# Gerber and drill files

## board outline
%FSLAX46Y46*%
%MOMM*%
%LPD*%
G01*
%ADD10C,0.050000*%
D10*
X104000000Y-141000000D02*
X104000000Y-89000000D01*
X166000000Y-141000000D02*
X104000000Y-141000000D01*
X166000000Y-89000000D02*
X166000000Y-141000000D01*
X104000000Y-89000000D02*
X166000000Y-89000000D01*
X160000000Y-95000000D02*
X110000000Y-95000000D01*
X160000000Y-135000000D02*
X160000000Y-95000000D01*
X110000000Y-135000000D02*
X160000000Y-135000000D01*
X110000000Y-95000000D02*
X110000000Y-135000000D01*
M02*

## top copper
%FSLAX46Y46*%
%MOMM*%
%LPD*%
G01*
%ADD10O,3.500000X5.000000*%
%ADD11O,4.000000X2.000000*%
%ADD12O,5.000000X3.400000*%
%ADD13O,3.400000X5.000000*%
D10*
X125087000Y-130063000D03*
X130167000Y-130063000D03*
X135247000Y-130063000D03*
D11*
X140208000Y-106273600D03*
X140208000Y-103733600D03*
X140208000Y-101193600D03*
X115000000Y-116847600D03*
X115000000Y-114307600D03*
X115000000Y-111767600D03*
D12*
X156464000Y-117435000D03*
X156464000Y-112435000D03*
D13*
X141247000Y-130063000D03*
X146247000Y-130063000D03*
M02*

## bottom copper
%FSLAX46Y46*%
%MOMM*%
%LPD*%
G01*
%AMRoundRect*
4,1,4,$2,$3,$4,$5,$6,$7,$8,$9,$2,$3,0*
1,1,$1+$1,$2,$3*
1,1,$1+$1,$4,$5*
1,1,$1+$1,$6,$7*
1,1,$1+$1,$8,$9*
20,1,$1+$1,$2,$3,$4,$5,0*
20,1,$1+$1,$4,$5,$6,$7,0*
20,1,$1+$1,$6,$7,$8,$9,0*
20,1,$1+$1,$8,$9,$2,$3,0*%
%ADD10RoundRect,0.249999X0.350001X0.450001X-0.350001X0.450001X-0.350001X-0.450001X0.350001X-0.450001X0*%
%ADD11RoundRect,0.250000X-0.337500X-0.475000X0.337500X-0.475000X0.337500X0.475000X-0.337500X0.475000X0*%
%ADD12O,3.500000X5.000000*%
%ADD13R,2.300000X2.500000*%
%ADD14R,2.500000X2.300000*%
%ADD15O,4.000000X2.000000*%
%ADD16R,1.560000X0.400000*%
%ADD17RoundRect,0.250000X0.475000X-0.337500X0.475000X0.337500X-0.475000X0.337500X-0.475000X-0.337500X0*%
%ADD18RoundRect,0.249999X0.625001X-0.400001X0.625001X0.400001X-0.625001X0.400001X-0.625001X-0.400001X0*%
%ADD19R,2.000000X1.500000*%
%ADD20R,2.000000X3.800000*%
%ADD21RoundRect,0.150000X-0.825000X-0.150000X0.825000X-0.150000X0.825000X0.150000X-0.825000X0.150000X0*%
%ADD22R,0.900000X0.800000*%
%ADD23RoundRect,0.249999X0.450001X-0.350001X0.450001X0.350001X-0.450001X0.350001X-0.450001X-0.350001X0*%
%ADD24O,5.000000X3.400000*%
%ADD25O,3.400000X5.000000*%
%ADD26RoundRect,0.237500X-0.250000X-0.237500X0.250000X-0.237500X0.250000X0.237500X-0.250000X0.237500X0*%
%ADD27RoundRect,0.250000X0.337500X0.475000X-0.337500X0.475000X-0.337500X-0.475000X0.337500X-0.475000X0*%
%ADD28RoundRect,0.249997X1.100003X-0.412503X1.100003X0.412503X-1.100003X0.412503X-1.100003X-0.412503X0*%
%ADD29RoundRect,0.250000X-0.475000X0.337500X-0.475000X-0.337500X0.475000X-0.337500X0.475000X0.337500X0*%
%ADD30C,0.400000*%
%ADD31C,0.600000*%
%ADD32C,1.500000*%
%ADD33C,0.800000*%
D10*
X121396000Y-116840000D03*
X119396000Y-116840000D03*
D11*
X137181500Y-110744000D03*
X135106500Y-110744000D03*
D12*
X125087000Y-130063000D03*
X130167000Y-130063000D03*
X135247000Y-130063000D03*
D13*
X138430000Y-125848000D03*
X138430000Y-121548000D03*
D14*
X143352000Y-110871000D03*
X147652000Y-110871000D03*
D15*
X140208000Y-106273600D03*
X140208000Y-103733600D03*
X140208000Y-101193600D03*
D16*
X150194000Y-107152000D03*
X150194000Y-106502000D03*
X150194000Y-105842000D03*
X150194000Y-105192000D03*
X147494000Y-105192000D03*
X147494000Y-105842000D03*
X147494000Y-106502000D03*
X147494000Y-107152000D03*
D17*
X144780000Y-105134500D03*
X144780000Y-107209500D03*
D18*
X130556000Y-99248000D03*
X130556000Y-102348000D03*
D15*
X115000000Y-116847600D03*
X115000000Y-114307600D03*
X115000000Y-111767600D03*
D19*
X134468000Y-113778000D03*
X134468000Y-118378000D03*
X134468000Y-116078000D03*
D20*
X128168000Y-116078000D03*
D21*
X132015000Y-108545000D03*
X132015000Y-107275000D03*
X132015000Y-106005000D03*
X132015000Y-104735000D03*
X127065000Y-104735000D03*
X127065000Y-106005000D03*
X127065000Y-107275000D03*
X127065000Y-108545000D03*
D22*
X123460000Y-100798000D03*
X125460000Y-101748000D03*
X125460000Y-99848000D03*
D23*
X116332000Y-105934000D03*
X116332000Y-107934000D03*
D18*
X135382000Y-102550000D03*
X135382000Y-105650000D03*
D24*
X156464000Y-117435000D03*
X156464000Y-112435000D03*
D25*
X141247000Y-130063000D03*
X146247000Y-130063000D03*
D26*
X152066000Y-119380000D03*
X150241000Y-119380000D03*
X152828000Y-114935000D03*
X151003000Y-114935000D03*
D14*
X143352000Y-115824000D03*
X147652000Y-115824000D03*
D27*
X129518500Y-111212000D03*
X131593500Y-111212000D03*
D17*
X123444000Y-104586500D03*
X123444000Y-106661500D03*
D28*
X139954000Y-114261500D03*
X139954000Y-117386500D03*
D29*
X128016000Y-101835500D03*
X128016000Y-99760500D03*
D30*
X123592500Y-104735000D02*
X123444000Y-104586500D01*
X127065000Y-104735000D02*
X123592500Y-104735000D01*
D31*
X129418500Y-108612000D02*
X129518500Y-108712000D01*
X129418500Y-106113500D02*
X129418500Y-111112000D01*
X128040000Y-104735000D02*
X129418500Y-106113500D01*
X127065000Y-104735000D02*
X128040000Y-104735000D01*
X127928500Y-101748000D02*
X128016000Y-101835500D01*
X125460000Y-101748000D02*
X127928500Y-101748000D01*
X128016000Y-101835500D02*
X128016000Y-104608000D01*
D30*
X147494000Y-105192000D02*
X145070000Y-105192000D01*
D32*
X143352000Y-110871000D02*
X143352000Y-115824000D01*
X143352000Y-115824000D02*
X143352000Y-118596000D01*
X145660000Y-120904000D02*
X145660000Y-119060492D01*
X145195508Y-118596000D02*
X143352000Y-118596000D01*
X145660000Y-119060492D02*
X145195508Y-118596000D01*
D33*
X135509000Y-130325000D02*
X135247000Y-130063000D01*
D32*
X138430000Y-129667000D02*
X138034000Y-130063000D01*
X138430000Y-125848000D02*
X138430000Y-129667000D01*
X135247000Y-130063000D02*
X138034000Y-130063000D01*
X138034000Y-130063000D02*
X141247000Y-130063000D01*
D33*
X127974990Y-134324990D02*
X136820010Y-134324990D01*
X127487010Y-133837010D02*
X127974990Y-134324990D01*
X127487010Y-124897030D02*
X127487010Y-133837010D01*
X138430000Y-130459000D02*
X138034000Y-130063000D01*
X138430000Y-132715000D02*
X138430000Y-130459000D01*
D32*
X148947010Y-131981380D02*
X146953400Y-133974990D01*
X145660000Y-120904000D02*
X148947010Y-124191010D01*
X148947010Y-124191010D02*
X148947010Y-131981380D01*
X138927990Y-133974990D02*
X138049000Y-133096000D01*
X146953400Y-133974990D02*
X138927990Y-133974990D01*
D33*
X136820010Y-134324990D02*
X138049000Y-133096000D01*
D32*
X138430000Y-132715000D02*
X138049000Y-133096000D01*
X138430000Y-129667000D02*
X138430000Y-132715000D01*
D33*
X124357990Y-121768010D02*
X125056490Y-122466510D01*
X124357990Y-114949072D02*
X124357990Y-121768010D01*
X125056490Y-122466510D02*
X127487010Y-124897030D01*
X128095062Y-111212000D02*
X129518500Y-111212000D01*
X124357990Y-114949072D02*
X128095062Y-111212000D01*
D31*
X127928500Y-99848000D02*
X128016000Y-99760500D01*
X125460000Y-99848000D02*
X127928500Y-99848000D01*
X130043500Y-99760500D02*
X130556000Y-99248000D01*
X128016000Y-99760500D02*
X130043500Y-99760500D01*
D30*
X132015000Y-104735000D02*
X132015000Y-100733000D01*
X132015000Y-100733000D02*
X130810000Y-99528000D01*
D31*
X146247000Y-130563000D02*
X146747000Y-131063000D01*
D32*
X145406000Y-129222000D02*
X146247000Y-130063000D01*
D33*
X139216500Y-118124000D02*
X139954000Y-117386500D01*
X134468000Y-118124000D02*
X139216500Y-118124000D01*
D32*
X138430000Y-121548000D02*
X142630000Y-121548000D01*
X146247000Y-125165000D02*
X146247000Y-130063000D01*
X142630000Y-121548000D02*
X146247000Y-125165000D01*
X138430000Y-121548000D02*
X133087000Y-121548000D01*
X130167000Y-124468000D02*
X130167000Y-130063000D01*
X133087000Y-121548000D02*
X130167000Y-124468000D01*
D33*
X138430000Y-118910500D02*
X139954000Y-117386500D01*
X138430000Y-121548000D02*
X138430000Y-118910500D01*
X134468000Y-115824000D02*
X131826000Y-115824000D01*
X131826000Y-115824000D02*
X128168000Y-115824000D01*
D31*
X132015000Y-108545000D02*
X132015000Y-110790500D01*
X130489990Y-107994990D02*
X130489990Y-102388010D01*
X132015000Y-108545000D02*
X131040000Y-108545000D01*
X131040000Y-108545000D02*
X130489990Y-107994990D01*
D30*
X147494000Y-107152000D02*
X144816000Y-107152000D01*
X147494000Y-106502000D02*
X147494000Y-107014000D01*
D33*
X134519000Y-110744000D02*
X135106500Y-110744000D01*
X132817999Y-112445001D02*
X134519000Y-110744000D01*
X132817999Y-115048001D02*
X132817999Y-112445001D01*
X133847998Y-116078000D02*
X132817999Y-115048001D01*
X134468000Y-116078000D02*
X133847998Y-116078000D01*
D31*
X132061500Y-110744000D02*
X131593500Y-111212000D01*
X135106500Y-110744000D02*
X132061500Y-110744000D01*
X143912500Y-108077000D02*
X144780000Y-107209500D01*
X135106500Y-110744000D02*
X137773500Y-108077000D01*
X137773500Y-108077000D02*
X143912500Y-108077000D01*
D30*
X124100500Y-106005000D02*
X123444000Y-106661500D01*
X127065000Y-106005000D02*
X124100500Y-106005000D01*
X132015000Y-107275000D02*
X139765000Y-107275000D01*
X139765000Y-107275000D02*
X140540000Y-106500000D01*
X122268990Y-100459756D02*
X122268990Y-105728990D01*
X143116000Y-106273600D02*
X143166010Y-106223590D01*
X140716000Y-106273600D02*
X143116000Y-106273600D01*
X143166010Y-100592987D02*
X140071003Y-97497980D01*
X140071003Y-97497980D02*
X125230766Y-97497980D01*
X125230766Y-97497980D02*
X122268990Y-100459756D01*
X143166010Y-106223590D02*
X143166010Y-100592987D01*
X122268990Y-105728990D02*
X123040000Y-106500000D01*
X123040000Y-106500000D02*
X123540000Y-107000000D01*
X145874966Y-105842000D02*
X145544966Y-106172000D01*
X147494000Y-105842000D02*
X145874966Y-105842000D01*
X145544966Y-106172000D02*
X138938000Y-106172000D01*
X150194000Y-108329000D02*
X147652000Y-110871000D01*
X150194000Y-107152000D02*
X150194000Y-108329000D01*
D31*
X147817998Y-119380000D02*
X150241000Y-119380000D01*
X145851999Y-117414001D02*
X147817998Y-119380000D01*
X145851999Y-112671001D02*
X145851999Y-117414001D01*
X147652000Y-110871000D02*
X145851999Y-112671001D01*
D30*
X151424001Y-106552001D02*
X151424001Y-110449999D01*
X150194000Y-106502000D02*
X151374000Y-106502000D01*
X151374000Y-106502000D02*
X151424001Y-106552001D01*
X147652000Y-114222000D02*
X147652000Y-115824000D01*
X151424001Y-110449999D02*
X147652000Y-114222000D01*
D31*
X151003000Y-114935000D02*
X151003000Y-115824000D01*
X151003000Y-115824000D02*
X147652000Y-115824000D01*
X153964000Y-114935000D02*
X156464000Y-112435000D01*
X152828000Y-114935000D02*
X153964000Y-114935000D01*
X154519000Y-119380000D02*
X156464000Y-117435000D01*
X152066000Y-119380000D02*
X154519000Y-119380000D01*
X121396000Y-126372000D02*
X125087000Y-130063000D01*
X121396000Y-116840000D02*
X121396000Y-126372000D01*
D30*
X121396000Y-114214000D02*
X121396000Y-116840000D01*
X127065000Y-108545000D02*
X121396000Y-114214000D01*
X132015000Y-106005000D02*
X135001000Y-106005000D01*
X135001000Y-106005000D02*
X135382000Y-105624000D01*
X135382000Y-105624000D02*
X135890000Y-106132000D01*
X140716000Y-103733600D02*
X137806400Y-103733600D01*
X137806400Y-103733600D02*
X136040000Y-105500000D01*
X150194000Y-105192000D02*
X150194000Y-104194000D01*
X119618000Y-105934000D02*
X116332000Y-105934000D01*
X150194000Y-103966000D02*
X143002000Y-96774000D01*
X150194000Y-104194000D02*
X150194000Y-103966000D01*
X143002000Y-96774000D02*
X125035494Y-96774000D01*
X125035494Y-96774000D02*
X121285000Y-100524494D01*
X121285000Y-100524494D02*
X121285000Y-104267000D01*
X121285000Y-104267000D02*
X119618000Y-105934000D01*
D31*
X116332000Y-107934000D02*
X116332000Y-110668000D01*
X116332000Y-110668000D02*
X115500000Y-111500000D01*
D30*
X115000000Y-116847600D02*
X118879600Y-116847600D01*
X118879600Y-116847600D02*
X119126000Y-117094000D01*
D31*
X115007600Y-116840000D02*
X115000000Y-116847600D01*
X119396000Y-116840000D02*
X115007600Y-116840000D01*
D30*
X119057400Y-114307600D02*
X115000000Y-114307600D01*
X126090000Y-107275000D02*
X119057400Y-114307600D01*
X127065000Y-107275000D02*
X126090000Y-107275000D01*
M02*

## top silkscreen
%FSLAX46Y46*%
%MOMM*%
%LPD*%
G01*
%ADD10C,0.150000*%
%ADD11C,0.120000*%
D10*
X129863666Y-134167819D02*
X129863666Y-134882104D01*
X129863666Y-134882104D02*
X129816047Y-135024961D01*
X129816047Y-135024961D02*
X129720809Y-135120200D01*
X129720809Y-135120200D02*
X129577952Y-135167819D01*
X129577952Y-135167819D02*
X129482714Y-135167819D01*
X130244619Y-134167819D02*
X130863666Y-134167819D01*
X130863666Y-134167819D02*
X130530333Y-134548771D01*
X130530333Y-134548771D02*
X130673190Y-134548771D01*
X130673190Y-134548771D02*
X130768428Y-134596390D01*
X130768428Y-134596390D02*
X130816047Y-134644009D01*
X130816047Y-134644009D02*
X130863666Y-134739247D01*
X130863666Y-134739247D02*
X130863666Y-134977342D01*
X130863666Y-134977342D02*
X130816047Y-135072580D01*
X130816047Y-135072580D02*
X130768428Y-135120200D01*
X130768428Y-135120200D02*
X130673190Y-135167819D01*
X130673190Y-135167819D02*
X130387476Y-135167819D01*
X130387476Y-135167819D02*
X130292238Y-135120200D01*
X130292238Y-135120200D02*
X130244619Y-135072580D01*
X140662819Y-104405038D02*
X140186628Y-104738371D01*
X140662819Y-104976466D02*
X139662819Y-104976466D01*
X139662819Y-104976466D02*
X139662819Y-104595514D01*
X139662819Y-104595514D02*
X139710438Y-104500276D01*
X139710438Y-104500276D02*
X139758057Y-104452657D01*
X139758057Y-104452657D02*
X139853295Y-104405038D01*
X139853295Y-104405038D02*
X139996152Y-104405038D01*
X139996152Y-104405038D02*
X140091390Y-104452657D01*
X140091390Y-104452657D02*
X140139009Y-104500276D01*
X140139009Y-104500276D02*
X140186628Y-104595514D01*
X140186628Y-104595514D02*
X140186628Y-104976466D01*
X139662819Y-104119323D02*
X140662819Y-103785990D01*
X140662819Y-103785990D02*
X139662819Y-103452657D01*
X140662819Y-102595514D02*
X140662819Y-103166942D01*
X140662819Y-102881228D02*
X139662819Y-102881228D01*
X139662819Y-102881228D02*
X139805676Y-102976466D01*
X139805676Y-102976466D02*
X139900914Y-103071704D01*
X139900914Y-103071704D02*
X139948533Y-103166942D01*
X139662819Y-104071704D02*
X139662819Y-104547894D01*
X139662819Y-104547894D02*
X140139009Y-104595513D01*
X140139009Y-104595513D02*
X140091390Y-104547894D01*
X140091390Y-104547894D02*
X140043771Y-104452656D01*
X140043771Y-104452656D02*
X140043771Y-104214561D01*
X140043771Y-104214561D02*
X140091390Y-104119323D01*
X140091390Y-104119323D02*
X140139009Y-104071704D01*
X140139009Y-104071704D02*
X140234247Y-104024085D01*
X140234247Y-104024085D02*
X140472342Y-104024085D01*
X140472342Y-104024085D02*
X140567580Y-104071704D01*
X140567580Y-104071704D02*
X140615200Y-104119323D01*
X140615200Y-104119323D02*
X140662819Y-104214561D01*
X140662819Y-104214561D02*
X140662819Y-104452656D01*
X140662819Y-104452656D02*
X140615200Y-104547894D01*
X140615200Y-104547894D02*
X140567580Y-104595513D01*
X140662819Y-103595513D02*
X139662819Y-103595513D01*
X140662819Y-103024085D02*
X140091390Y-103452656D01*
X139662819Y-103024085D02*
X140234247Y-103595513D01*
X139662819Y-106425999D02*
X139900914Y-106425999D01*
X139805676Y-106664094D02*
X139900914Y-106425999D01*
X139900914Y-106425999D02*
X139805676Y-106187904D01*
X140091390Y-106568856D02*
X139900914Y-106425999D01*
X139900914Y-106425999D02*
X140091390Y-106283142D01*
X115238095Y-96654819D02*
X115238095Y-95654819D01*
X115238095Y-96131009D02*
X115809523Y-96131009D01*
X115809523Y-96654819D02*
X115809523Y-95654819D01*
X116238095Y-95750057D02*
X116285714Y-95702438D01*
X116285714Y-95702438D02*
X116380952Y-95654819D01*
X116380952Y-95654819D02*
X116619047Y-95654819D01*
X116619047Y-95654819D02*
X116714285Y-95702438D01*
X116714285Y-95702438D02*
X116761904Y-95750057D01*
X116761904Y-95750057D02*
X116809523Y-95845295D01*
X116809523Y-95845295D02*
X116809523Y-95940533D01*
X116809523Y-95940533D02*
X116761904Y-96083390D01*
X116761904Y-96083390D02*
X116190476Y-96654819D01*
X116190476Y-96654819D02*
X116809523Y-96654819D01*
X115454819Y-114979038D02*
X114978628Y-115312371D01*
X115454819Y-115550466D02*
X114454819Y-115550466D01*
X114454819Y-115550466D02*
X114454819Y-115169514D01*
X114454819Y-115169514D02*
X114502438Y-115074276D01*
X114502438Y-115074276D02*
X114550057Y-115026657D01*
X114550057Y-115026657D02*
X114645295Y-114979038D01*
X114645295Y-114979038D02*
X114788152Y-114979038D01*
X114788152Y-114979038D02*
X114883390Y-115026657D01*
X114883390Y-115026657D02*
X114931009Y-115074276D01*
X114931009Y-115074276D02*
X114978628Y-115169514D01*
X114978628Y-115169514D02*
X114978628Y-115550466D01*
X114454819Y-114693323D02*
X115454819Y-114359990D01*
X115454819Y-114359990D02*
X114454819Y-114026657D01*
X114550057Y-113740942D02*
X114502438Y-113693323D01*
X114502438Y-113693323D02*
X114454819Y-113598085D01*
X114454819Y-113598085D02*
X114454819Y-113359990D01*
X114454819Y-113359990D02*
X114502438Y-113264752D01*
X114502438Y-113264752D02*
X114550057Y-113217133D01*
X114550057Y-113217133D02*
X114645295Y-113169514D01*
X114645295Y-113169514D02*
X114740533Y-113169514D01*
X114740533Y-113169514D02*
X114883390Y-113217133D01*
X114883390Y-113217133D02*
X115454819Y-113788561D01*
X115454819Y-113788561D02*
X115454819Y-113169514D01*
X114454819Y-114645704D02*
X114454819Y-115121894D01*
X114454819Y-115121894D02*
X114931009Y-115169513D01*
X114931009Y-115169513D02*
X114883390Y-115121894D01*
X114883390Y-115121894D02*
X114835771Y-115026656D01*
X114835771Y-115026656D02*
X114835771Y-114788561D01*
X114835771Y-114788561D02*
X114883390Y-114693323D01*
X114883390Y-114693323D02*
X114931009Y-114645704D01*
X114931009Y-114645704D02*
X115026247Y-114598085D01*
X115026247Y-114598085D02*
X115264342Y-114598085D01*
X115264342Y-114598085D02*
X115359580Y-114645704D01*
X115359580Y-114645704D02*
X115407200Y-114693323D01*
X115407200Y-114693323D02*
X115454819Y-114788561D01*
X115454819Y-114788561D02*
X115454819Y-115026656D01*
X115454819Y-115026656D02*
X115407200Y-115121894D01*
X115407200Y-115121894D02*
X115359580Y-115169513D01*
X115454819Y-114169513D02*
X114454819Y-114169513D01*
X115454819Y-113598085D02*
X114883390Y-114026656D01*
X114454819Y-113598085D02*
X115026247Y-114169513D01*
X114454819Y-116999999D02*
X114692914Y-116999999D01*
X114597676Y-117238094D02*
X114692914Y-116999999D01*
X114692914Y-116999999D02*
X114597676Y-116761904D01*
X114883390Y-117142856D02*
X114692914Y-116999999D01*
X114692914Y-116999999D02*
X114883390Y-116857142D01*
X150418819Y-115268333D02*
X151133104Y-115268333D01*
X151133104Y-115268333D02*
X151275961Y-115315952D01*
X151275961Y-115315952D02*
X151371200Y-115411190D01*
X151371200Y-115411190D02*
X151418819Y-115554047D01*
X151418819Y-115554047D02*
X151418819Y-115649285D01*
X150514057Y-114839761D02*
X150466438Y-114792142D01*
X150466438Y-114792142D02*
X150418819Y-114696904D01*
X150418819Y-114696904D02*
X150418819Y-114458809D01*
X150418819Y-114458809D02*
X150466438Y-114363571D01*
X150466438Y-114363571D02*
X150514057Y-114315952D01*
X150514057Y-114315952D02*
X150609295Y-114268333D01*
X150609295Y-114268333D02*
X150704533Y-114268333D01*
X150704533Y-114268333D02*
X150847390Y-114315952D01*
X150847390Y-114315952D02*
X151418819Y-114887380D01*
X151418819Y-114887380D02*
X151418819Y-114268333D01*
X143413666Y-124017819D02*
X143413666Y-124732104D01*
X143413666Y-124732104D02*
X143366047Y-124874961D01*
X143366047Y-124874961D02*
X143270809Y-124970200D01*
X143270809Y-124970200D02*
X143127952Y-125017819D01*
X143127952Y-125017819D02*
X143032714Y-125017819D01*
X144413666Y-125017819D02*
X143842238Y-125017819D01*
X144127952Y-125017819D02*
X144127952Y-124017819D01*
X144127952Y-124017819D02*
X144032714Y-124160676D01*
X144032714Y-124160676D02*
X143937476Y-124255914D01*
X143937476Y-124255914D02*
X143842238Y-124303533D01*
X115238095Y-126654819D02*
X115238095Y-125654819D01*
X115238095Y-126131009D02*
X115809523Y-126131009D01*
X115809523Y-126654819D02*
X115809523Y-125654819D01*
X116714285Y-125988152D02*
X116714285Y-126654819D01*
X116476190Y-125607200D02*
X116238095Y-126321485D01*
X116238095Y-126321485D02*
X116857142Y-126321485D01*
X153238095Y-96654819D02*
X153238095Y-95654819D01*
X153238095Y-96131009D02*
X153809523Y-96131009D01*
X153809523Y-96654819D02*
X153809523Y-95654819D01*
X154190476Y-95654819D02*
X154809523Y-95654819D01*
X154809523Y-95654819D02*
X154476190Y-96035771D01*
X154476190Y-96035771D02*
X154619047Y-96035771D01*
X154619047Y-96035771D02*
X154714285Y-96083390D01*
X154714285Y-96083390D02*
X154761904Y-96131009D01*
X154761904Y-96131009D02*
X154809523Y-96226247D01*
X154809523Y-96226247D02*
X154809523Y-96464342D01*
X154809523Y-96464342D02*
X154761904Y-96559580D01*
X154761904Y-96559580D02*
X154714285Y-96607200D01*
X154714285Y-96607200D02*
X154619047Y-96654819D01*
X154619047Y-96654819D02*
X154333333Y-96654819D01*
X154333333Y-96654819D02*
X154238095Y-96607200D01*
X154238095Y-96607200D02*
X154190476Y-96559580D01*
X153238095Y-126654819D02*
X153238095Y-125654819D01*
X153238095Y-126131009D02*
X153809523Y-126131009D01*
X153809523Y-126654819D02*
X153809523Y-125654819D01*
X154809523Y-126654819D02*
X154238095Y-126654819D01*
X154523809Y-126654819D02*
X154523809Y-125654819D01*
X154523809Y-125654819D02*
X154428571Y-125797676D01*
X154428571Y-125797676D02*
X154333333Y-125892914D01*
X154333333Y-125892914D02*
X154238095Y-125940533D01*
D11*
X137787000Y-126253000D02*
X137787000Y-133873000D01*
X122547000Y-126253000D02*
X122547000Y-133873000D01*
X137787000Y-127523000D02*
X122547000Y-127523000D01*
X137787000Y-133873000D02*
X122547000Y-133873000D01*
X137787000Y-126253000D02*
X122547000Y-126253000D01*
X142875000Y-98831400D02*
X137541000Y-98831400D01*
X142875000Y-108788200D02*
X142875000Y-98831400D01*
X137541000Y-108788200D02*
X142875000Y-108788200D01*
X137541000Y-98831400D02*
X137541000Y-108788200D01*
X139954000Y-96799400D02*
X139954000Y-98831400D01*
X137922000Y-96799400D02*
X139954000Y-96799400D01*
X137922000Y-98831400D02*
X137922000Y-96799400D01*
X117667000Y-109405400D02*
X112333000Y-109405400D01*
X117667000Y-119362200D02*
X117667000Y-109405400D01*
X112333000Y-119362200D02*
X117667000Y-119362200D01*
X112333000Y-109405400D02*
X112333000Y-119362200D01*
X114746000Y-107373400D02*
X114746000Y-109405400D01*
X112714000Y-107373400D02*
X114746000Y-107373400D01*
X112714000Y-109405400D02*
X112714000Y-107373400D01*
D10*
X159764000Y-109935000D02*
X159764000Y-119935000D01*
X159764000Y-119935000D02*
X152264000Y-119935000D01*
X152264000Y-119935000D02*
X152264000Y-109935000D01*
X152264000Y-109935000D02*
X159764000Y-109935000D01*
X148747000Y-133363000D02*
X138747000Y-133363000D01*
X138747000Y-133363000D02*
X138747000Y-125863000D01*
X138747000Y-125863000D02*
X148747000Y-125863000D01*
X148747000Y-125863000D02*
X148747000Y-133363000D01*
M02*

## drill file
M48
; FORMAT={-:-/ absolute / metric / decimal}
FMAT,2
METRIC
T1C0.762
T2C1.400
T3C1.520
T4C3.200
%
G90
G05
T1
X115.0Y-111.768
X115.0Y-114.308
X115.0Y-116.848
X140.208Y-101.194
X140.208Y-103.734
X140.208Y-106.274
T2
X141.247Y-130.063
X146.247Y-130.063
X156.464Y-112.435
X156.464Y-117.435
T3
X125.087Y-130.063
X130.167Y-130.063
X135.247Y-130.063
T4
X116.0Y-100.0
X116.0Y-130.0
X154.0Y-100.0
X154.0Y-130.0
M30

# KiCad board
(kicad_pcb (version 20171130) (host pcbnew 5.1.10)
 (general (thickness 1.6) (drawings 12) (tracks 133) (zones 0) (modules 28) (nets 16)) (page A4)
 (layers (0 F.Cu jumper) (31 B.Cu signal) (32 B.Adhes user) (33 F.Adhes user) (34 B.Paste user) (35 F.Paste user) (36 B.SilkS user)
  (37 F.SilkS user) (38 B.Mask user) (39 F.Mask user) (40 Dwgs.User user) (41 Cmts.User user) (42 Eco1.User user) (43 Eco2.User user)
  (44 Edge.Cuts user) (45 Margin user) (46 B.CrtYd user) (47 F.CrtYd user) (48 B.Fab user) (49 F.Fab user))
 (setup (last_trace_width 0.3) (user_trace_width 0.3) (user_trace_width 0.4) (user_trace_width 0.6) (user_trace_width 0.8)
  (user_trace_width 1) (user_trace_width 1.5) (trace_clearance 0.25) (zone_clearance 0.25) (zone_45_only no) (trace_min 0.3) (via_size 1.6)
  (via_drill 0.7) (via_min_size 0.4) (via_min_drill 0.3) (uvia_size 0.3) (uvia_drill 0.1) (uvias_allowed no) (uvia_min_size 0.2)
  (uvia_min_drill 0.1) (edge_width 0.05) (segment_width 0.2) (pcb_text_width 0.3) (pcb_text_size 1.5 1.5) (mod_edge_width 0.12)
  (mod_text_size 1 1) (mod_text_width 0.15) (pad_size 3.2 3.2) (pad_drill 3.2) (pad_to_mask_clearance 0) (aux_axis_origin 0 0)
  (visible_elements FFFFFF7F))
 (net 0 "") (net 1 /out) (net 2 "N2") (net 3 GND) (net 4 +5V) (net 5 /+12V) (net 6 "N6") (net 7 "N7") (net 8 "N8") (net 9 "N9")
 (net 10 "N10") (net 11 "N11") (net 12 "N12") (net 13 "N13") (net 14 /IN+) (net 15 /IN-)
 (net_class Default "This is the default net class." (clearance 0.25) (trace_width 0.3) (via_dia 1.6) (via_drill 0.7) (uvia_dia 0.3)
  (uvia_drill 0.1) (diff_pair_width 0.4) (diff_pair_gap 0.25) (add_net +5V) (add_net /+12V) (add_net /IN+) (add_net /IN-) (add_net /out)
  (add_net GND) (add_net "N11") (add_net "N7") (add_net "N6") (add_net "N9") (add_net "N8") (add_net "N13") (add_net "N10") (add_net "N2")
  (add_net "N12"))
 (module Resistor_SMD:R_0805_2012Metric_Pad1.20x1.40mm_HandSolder (layer B.Cu) (at 120.396 116.84 180)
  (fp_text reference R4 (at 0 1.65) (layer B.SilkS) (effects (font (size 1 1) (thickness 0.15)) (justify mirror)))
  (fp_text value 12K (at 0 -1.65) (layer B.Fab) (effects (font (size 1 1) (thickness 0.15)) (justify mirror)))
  (pad 1 smd roundrect (at -1 0 180) (size 1.2 1.4) (layers B.Cu B.Paste B.Mask) (roundrect_rratio 0.2083325) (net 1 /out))
  (pad 2 smd roundrect (at 1 0 180) (size 1.2 1.4) (layers B.Cu B.Paste B.Mask) (roundrect_rratio 0.2083325) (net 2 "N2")))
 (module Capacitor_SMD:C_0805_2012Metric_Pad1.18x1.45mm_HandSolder (layer B.Cu) (at 136.144 110.744)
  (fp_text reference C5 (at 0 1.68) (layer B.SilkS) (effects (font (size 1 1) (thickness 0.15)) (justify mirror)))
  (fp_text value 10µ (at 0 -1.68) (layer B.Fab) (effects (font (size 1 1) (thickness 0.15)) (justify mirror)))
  (pad 2 smd roundrect (at 1.0375 0) (size 1.175 1.45) (layers B.Cu B.Paste B.Mask) (roundrect_rratio 0.2127659574468085) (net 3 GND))
  (pad 1 smd roundrect (at -1.0375 0) (size 1.175 1.45) (layers B.Cu B.Paste B.Mask) (roundrect_rratio 0.2127659574468085) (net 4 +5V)))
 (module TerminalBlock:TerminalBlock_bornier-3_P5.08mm (layer F.Cu) (at 135.247 130.063 180)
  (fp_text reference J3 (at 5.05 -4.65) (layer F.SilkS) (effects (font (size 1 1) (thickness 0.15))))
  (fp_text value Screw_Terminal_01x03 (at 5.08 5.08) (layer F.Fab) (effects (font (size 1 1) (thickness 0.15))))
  (fp_line (start -2.54 3.81) (end -2.54 -3.81) (layer F.SilkS) (width 0.12))
  (fp_line (start 12.7 3.81) (end 12.7 -3.81) (layer F.SilkS) (width 0.12))
  (fp_line (start -2.54 2.54) (end 12.7 2.54) (layer F.SilkS) (width 0.12))
  (fp_line (start -2.54 -3.81) (end 12.7 -3.81) (layer F.SilkS) (width 0.12))
  (fp_line (start -2.54 3.81) (end 12.7 3.81) (layer F.SilkS) (width 0.12))
  (pad 3 thru_hole oval (at 10.16 0 180) (size 3.5 5) (drill 1.52) (layers *.Cu *.Mask) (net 1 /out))
  (pad 2 thru_hole oval (at 5.08 0 180) (size 3.5 5) (drill 1.52) (layers *.Cu *.Mask) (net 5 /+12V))
  (pad 1 thru_hole oval (at 0 0 180) (size 3.5 5) (drill 1.52) (layers *.Cu *.Mask) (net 3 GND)))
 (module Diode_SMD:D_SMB (layer B.Cu) (at 138.43 123.698 270)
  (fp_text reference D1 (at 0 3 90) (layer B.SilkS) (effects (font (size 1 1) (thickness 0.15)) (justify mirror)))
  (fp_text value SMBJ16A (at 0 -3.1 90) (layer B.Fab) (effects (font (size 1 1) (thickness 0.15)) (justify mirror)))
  (pad 2 smd rect (at 2.15 0 270) (size 2.5 2.3) (layers B.Cu B.Paste B.Mask) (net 3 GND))
  (pad 1 smd rect (at -2.15 0 270) (size 2.5 2.3) (layers B.Cu B.Paste B.Mask) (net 5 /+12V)))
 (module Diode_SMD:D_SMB (layer B.Cu) (at 145.502 110.871 180)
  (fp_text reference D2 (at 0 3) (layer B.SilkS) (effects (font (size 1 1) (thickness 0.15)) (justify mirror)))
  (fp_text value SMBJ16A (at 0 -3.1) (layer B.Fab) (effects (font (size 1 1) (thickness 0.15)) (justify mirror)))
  (pad 2 smd rect (at 2.15 0 180) (size 2.5 2.3) (layers B.Cu B.Paste B.Mask) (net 3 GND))
  (pad 1 smd rect (at -2.15 0 180) (size 2.5 2.3) (layers B.Cu B.Paste B.Mask) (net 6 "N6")))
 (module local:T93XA (layer F.Cu) (at 140.208 106.426 270)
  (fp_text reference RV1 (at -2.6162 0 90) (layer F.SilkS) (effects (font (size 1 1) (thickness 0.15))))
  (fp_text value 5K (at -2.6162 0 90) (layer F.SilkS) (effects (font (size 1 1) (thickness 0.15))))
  (fp_line (start -7.5946 -2.667) (end -7.5946 2.667) (layer F.SilkS) (width 0.12))
  (fp_line (start 2.3622 -2.667) (end -7.5946 -2.667) (layer F.SilkS) (width 0.12))
  (fp_line (start 2.3622 2.667) (end 2.3622 -2.667) (layer F.SilkS) (width 0.12))
  (fp_line (start -7.5946 2.667) (end 2.3622 2.667) (layer F.SilkS) (width 0.12))
  (fp_line (start -9.6266 0.254) (end -7.5946 0.254) (layer F.SilkS) (width 0.12))
  (fp_line (start -9.6266 2.286) (end -9.6266 0.254) (layer F.SilkS) (width 0.12))
  (fp_line (start -7.5946 2.286) (end -9.6266 2.286) (layer F.SilkS) (width 0.12))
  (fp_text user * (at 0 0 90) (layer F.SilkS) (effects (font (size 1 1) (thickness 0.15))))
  (pad 3 thru_hole oval (at -0.1524 0 270) (size 2 4) (drill 0.762) (layers *.Cu *.Mask) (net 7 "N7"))
  (pad 2 thru_hole oval (at -2.6924 0 270) (size 2 4) (drill 0.762) (layers *.Cu *.Mask) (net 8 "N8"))
  (pad 1 thru_hole oval (at -5.2324 0 270) (size 2 4) (drill 0.762) (layers *.Cu *.Mask)))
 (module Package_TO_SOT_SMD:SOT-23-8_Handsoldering (layer B.Cu) (at 148.844 106.172)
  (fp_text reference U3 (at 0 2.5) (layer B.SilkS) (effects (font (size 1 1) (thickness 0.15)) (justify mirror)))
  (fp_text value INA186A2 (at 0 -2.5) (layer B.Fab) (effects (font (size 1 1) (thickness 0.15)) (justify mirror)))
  (pad 8 smd rect (at 1.35 0.98) (size 1.56 0.4) (layers B.Cu B.Paste B.Mask) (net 6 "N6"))
  (pad 7 smd rect (at 1.35 0.33) (size 1.56 0.4) (layers B.Cu B.Paste B.Mask) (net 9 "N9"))
  (pad 6 smd rect (at 1.35 -0.33) (size 1.56 0.4) (layers B.Cu B.Paste B.Mask))
  (pad 5 smd rect (at 1.35 -0.98) (size 1.56 0.4) (layers B.Cu B.Paste B.Mask) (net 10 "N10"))
  (pad 4 smd rect (at -1.35 -0.98) (size 1.56 0.4) (layers B.Cu B.Paste B.Mask) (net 3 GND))
  (pad 3 smd rect (at -1.35 -0.33) (size 1.56 0.4) (layers B.Cu B.Paste B.Mask) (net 7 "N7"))
  (pad 2 smd rect (at -1.35 0.33) (size 1.56 0.4) (layers B.Cu B.Paste B.Mask) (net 4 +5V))
  (pad 1 smd rect (at -1.35 0.98) (size 1.56 0.4) (layers B.Cu B.Paste B.Mask) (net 4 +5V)))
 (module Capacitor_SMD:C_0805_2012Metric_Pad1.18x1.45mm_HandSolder (layer B.Cu) (at 144.78 106.172 90)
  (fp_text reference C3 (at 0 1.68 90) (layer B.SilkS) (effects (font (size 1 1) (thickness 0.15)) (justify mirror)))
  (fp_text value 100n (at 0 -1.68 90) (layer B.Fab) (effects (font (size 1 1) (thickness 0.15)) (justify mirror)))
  (pad 2 smd roundrect (at 1.0375 0 90) (size 1.175 1.45) (layers B.Cu B.Paste B.Mask) (roundrect_rratio 0.2127659574468085) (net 3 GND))
  (pad 1 smd roundrect (at -1.0375 0 90) (size 1.175 1.45) (layers B.Cu B.Paste B.Mask) (roundrect_rratio 0.2127659574468085) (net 4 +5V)))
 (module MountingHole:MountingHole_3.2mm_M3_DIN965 (layer F.Cu) (at 116 100)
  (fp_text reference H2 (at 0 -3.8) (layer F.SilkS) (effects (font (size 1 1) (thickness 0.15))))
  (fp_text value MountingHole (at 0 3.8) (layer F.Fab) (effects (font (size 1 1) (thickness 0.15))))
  (pad 1 np_thru_hole circle (at 0 0) (size 3.2 3.2) (drill 3.2) (layers *.Cu *.Mask)))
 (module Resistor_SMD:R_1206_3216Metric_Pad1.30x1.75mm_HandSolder (layer B.Cu) (at 130.556 100.798 90)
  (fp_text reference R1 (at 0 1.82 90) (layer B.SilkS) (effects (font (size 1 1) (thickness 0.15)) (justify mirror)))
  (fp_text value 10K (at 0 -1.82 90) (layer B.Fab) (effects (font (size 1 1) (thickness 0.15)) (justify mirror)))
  (pad 2 smd roundrect (at 1.55 0 90) (size 1.3 1.75) (layers B.Cu B.Paste B.Mask) (roundrect_rratio 0.1923069230769231) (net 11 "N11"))
  (pad 1 smd roundrect (at -1.55 0 90) (size 1.3 1.75) (layers B.Cu B.Paste B.Mask) (roundrect_rratio 0.1923069230769231) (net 4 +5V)))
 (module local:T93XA (layer F.Cu) (at 115 117 270)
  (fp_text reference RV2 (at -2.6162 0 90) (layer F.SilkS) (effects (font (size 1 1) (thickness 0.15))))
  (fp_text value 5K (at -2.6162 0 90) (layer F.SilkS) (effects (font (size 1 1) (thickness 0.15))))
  (fp_line (start -7.5946 -2.667) (end -7.5946 2.667) (layer F.SilkS) (width 0.12))
  (fp_line (start 2.3622 -2.667) (end -7.5946 -2.667) (layer F.SilkS) (width 0.12))
  (fp_line (start 2.3622 2.667) (end 2.3622 -2.667) (layer F.SilkS) (width 0.12))
  (fp_line (start -7.5946 2.667) (end 2.3622 2.667) (layer F.SilkS) (width 0.12))
  (fp_line (start -9.6266 0.254) (end -7.5946 0.254) (layer F.SilkS) (width 0.12))
  (fp_line (start -9.6266 2.286) (end -9.6266 0.254) (layer F.SilkS) (width 0.12))
  (fp_line (start -7.5946 2.286) (end -9.6266 2.286) (layer F.SilkS) (width 0.12))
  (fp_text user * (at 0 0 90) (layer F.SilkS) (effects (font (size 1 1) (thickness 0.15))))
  (pad 3 thru_hole oval (at -0.1524 0 270) (size 2 4) (drill 0.762) (layers *.Cu *.Mask) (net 2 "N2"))
  (pad 2 thru_hole oval (at -2.6924 0 270) (size 2 4) (drill 0.762) (layers *.Cu *.Mask) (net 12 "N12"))
  (pad 1 thru_hole oval (at -5.2324 0 270) (size 2 4) (drill 0.762) (layers *.Cu *.Mask) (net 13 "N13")))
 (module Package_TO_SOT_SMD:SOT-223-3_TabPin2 (layer B.Cu) (at 131.318 116.078 180)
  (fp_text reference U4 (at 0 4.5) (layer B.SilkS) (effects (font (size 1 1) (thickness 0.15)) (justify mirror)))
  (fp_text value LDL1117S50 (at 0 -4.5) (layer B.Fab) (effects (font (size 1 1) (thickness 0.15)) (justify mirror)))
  (pad 1 smd rect (at -3.15 2.3 180) (size 2 1.5) (layers B.Cu B.Paste B.Mask) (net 3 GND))
  (pad 3 smd rect (at -3.15 -2.3 180) (size 2 1.5) (layers B.Cu B.Paste B.Mask) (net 5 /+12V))
  (pad 2 smd rect (at -3.15 0 180) (size 2 1.5) (layers B.Cu B.Paste B.Mask) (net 4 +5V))
  (pad 2 smd rect (at 3.15 0 180) (size 2 3.8) (layers B.Cu B.Paste B.Mask) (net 4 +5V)))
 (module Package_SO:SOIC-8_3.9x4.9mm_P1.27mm (layer B.Cu) (at 129.54 106.64)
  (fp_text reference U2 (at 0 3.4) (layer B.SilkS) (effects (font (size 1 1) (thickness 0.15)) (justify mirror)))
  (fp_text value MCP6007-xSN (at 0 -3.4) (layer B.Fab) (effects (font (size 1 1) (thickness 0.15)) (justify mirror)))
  (pad 8 smd roundrect (at 2.475 1.905) (size 1.95 0.6) (layers B.Cu B.Paste B.Mask) (roundrect_rratio 0.25) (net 4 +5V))
  (pad 7 smd roundrect (at 2.475 0.635) (size 1.95 0.6) (layers B.Cu B.Paste B.Mask) (roundrect_rratio 0.25) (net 7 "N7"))
  (pad 6 smd roundrect (at 2.475 -0.635) (size 1.95 0.6) (layers B.Cu B.Paste B.Mask) (roundrect_rratio 0.25) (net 8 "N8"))
  (pad 5 smd roundrect (at 2.475 -1.905) (size 1.95 0.6) (layers B.Cu B.Paste B.Mask) (roundrect_rratio 0.25) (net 11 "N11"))
  (pad 4 smd roundrect (at -2.475 -1.905) (size 1.95 0.6) (layers B.Cu B.Paste B.Mask) (roundrect_rratio 0.25) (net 3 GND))
  (pad 3 smd roundrect (at -2.475 -0.635) (size 1.95 0.6) (layers B.Cu B.Paste B.Mask) (roundrect_rratio 0.25) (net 7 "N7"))
  (pad 2 smd roundrect (at -2.475 0.635) (size 1.95 0.6) (layers B.Cu B.Paste B.Mask) (roundrect_rratio 0.25) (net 12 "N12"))
  (pad 1 smd roundrect (at -2.475 1.905) (size 1.95 0.6) (layers B.Cu B.Paste B.Mask) (roundrect_rratio 0.25) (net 1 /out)))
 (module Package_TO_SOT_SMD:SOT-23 (layer B.Cu) (at 124.46 100.798 180)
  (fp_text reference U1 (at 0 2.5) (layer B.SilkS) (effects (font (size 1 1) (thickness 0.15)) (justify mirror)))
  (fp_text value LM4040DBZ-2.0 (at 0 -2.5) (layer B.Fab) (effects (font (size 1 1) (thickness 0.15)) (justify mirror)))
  (pad 3 smd rect (at 1 0 180) (size 0.9 0.8) (layers B.Cu B.Paste B.Mask))
  (pad 2 smd rect (at -1 -0.95 180) (size 0.9 0.8) (layers B.Cu B.Paste B.Mask) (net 3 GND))
  (pad 1 smd rect (at -1 0.95 180) (size 0.9 0.8) (layers B.Cu B.Paste B.Mask) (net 11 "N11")))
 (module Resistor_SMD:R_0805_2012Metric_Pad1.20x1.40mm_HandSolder (layer B.Cu) (at 116.332 106.934 90)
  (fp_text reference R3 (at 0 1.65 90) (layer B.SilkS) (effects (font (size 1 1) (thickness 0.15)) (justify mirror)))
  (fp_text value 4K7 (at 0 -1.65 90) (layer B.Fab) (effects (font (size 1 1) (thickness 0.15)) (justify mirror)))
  (pad 2 smd roundrect (at 1 0 90) (size 1.2 1.4) (layers B.Cu B.Paste B.Mask) (roundrect_rratio 0.2083325) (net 10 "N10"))
  (pad 1 smd roundrect (at -1 0 90) (size 1.2 1.4) (layers B.Cu B.Paste B.Mask) (roundrect_rratio 0.2083325) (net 13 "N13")))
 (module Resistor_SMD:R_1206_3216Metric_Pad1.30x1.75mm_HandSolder (layer B.Cu) (at 135.382 104.1 90)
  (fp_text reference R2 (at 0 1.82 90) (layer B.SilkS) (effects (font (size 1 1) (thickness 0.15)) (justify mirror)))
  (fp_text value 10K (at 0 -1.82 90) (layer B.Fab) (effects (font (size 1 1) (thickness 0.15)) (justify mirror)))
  (pad 2 smd roundrect (at 1.55 0 90) (size 1.3 1.75) (layers B.Cu B.Paste B.Mask) (roundrect_rratio 0.1923069230769231) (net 3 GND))
  (pad 1 smd roundrect (at -1.55 0 90) (size 1.3 1.75) (layers B.Cu B.Paste B.Mask) (roundrect_rratio 0.1923069230769231) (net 8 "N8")))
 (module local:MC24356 (layer F.Cu) (at 156.464 114.935 270)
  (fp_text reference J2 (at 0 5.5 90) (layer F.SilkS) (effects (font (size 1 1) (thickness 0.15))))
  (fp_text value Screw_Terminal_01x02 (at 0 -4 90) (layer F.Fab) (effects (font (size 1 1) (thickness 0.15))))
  (fp_line (start -5 -3.3) (end 5 -3.3) (layer F.SilkS) (width 0.15))
  (fp_line (start 5 -3.3) (end 5 4.2) (layer F.SilkS) (width 0.15))
  (fp_line (start 5 4.2) (end -5 4.2) (layer F.SilkS) (width 0.15))
  (fp_line (start -5 4.2) (end -5 -3.3) (layer F.SilkS) (width 0.15))
  (pad 2 thru_hole oval (at 2.5 0 270) (size 3.4 5) (drill 1.4) (layers *.Cu *.Mask) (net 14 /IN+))
  (pad 1 thru_hole oval (at -2.5 0 270) (size 3.4 5) (drill 1.4) (layers *.Cu *.Mask) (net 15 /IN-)))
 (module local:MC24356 (layer F.Cu) (at 143.747 130.063 180)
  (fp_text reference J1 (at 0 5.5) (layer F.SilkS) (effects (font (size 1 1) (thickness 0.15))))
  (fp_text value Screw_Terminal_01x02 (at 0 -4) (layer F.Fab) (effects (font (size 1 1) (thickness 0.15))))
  (fp_line (start -5 -3.3) (end 5 -3.3) (layer F.SilkS) (width 0.15))
  (fp_line (start 5 -3.3) (end 5 4.2) (layer F.SilkS) (width 0.15))
  (fp_line (start 5 4.2) (end -5 4.2) (layer F.SilkS) (width 0.15))
  (fp_line (start -5 4.2) (end -5 -3.3) (layer F.SilkS) (width 0.15))
  (pad 2 thru_hole oval (at 2.5 0 180) (size 3.4 5) (drill 1.4) (layers *.Cu *.Mask) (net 3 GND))
  (pad 1 thru_hole oval (at -2.5 0 180) (size 3.4 5) (drill 1.4) (layers *.Cu *.Mask) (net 5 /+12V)))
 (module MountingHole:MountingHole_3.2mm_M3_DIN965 (layer F.Cu) (at 116 130)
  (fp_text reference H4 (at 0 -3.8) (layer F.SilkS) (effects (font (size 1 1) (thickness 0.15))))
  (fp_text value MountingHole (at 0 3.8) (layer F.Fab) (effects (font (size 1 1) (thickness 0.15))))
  (pad 1 np_thru_hole circle (at 0 0) (size 3.2 3.2) (drill 3.2) (layers *.Cu *.Mask)))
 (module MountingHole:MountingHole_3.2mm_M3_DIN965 (layer F.Cu) (at 154 100)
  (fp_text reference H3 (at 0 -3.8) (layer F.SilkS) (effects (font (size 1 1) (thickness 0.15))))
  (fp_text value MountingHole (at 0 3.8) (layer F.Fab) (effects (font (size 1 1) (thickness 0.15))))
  (pad 1 np_thru_hole circle (at 0 0) (size 3.2 3.2) (drill 3.2) (layers *.Cu *.Mask)))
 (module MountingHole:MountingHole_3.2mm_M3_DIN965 (layer F.Cu) (at 154 130)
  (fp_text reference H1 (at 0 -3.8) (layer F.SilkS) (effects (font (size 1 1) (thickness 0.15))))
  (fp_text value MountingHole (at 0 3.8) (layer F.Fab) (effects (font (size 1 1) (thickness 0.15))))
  (pad 1 np_thru_hole circle (at 0 0) (size 3.2 3.2) (drill 3.2) (layers *.Cu *.Mask)))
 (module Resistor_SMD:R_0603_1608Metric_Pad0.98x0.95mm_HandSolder (layer B.Cu) (at 151.1535 119.38)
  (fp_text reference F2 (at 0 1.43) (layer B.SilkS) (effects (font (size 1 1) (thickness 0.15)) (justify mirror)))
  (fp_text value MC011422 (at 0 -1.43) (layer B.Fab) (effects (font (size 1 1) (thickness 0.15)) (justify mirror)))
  (pad 2 smd roundrect (at 0.9125 0) (size 0.975 0.95) (layers B.Cu B.Paste B.Mask) (roundrect_rratio 0.25) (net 14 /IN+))
  (pad 1 smd roundrect (at -0.9125 0) (size 0.975 0.95) (layers B.Cu B.Paste B.Mask) (roundrect_rratio 0.25) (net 6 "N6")))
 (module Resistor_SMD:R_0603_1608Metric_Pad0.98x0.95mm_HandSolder (layer B.Cu) (at 151.9155 114.935)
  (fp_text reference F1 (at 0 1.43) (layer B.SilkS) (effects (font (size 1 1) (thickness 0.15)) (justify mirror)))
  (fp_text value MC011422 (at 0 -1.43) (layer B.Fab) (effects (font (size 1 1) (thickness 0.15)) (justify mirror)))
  (pad 2 smd roundrect (at 0.9125 0) (size 0.975 0.95) (layers B.Cu B.Paste B.Mask) (roundrect_rratio 0.25) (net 15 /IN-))
  (pad 1 smd roundrect (at -0.9125 0) (size 0.975 0.95) (layers B.Cu B.Paste B.Mask) (roundrect_rratio 0.25) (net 9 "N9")))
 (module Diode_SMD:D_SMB (layer B.Cu) (at 145.502 115.824 180)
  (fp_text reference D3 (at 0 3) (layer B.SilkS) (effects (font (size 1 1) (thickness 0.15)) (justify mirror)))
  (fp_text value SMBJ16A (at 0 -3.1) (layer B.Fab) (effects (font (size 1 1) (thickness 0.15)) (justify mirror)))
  (pad 2 smd rect (at 2.15 0 180) (size 2.5 2.3) (layers B.Cu B.Paste B.Mask) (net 3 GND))
  (pad 1 smd rect (at -2.15 0 180) (size 2.5 2.3) (layers B.Cu B.Paste B.Mask) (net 9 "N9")))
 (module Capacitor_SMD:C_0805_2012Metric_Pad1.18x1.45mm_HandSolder (layer B.Cu) (at 130.556 111.212 180)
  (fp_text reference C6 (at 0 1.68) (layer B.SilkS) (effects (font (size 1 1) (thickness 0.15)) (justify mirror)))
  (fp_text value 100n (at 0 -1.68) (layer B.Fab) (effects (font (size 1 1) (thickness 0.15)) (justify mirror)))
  (pad 2 smd roundrect (at 1.0375 0 180) (size 1.175 1.45) (layers B.Cu B.Paste B.Mask) (roundrect_rratio 0.2127659574468085) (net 3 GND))
  (pad 1 smd roundrect (at -1.0375 0 180) (size 1.175 1.45) (layers B.Cu B.Paste B.Mask) (roundrect_rratio 0.2127659574468085) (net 4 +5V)))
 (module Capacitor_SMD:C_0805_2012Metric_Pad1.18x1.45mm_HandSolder (layer B.Cu) (at 123.444 105.624 90)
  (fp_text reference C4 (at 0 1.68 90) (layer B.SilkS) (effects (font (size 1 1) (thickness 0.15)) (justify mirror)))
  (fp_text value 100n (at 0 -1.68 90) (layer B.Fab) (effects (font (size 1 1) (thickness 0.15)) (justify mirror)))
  (pad 2 smd roundrect (at 1.0375 0 90) (size 1.175 1.45) (layers B.Cu B.Paste B.Mask) (roundrect_rratio 0.2127659574468085) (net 3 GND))
  (pad 1 smd roundrect (at -1.0375 0 90) (size 1.175 1.45) (layers B.Cu B.Paste B.Mask) (roundrect_rratio 0.2127659574468085) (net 7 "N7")))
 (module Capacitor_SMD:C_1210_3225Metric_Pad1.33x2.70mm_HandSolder (layer B.Cu) (at 139.954 115.824 90)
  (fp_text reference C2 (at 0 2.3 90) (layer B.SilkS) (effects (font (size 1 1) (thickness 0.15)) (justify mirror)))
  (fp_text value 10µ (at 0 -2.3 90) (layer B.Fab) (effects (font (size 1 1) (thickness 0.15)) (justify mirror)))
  (pad 2 smd roundrect (at 1.5625 0 90) (size 1.325 2.7) (layers B.Cu B.Paste B.Mask) (roundrect_rratio 0.1886769811320755) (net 3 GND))
  (pad 1 smd roundrect (at -1.5625 0 90) (size 1.325 2.7) (layers B.Cu B.Paste B.Mask) (roundrect_rratio 0.1886769811320755) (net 5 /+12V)))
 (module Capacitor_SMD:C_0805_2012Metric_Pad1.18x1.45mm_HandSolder (layer B.Cu) (at 128.016 100.798 270)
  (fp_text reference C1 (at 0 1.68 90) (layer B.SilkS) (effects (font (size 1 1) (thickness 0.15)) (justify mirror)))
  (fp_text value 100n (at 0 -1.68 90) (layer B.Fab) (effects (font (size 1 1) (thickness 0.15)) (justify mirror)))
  (pad 2 smd roundrect (at 1.0375 0 270) (size 1.175 1.45) (layers B.Cu B.Paste B.Mask) (roundrect_rratio 0.2127659574468085) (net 3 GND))
  (pad 1 smd roundrect (at -1.0375 0 270) (size 1.175 1.45) (layers B.Cu B.Paste B.Mask) (roundrect_rratio 0.2127659574468085)
   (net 11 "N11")))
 (gr_line (start 104 141) (end 104 89) (layer Edge.Cuts) (width 0.05))
 (gr_line (start 166 141) (end 104 141) (layer Edge.Cuts) (width 0.05))
 (gr_line (start 166 89) (end 166 141) (layer Edge.Cuts) (width 0.05))
 (gr_line (start 104 89) (end 166 89) (layer Edge.Cuts) (width 0.05))
 (gr_line (start 160 95) (end 110 95) (layer Edge.Cuts) (width 0.05))
 (gr_line (start 160 135) (end 160 95) (layer Edge.Cuts) (width 0.05))
 (gr_line (start 110 135) (end 160 135) (layer Edge.Cuts) (width 0.05))
 (gr_line (start 110 95) (end 110 135) (layer Edge.Cuts) (width 0.05))
 (segment (start 123.5925 104.735) (end 123.444 104.5865) (width 0.4) (layer B.Cu) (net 3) (status 30))
 (segment (start 127.065 104.735) (end 123.5925 104.735) (width 0.4) (layer B.Cu) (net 3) (status 30))
 (segment (start 129.4185 108.612) (end 129.5185 108.712) (width 0.6) (layer B.Cu) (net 3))
 (segment (start 129.4185 106.1135) (end 129.4185 111.112) (width 0.6) (layer B.Cu) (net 3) (status 20))
 (segment (start 128.04 104.735) (end 129.4185 106.1135) (width 0.6) (layer B.Cu) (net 3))
 (segment (start 127.065 104.735) (end 128.04 104.735) (width 0.6) (layer B.Cu) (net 3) (status 10))
 (segment (start 127.9285 101.748) (end 128.016 101.8355) (width 0.6) (layer B.Cu) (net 3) (status 30))
 (segment (start 125.46 101.748) (end 127.9285 101.748) (width 0.6) (layer B.Cu) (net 3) (status 30))
 (segment (start 128.016 101.8355) (end 128.016 104.608) (width 0.6) (layer B.Cu) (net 3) (status 30))
 (segment (start 147.494 105.192) (end 145.07 105.192) (width 0.4) (layer B.Cu) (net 3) (status 30))
 (segment (start 143.352 110.871) (end 143.352 115.824) (width 1.5) (layer B.Cu) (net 3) (status 30))
 (segment (start 143.352 115.824) (end 143.352 118.596) (width 1.5) (layer B.Cu) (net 3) (status 10))
 (segment (start 145.66 120.904) (end 145.66 119.060492) (width 1.5) (layer B.Cu) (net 3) (status 10))
 (segment (start 145.195508 118.596) (end 143.352 118.596) (width 1.5) (layer B.Cu) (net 3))
 (segment (start 145.66 119.060492) (end 145.195508 118.596) (width 1.5) (layer B.Cu) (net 3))
 (segment (start 135.509 130.325) (end 135.247 130.063) (width 0.8) (layer B.Cu) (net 3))
 (segment (start 138.43 129.667) (end 138.034 130.063) (width 1.5) (layer B.Cu) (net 3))
 (segment (start 138.43 125.848) (end 138.43 129.667) (width 1.5) (layer B.Cu) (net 3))
 (segment (start 135.247 130.063) (end 138.034 130.063) (width 1.5) (layer B.Cu) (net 3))
 (segment (start 138.034 130.063) (end 141.247 130.063) (width 1.5) (layer B.Cu) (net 3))
 (segment (start 127.97499 134.32499) (end 136.82001 134.32499) (width 0.8) (layer B.Cu) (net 3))
 (segment (start 127.48701 133.83701) (end 127.97499 134.32499) (width 0.8) (layer B.Cu) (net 3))
 (segment (start 127.48701 124.89703) (end 127.48701 133.83701) (width 0.8) (layer B.Cu) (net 3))
 (segment (start 138.43 130.459) (end 138.034 130.063) (width 0.8) (layer B.Cu) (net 3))
 (segment (start 138.43 132.715) (end 138.43 130.459) (width 0.8) (layer B.Cu) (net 3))
 (segment (start 148.94701 131.98138) (end 146.9534 133.97499) (width 1.5) (layer B.Cu) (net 3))
 (segment (start 145.66 120.904) (end 148.94701 124.19101) (width 1.5) (layer B.Cu) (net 3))
 (segment (start 148.94701 124.19101) (end 148.94701 131.98138) (width 1.5) (layer B.Cu) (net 3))
 (segment (start 138.92799 133.97499) (end 138.049 133.096) (width 1.5) (layer B.Cu) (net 3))
 (segment (start 146.9534 133.97499) (end 138.92799 133.97499) (width 1.5) (layer B.Cu) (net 3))
 (segment (start 136.82001 134.32499) (end 138.049 133.096) (width 0.8) (layer B.Cu) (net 3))
 (segment (start 138.43 132.715) (end 138.049 133.096) (width 1.5) (layer B.Cu) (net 3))
 (segment (start 138.43 129.667) (end 138.43 132.715) (width 1.5) (layer B.Cu) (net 3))
 (segment (start 124.35799 121.76801) (end 125.05649 122.46651) (width 0.8) (layer B.Cu) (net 3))
 (segment (start 124.35799 114.949072) (end 124.35799 121.76801) (width 0.8) (layer B.Cu) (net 3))
 (segment (start 125.05649 122.46651) (end 127.48701 124.89703) (width 0.8) (layer B.Cu) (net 3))
 (segment (start 128.095062 111.212) (end 129.5185 111.212) (width 0.8) (layer B.Cu) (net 3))
 (segment (start 124.35799 114.949072) (end 128.095062 111.212) (width 0.8) (layer B.Cu) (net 3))
 (segment (start 127.9285 99.848) (end 128.016 99.7605) (width 0.6) (layer B.Cu) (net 11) (status 30))
 (segment (start 125.46 99.848) (end 127.9285 99.848) (width 0.6) (layer B.Cu) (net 11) (status 30))
 (segment (start 130.0435 99.7605) (end 130.556 99.248) (width 0.6) (layer B.Cu) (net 11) (status 30))
 (segment (start 128.016 99.7605) (end 130.0435 99.7605) (width 0.6) (layer B.Cu) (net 11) (status 30))
 (segment (start 132.015 104.735) (end 132.015 100.733) (width 0.4) (layer B.Cu) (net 11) (status 10))
 (segment (start 132.015 100.733) (end 130.81 99.528) (width 0.4) (layer B.Cu) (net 11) (status 20))
 (segment (start 146.247 130.563) (end 146.747 131.063) (width 0.6) (layer B.Cu) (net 5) (status 30))
 (segment (start 145.406 129.222) (end 146.247 130.063) (width 1.5) (layer B.Cu) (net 5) (status 30))
 (segment (start 139.2165 118.124) (end 139.954 117.3865) (width 0.8) (layer B.Cu) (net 5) (status 20))
 (segment (start 134.468 118.124) (end 139.2165 118.124) (width 0.8) (layer B.Cu) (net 5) (status 10))
 (segment (start 138.43 121.548) (end 142.63 121.548) (width 1.5) (layer B.Cu) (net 5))
 (segment (start 146.247 125.165) (end 146.247 130.063) (width 1.5) (layer B.Cu) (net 5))
 (segment (start 142.63 121.548) (end 146.247 125.165) (width 1.5) (layer B.Cu) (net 5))
 (segment (start 138.43 121.548) (end 133.087 121.548) (width 1.5) (layer B.Cu) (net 5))
 (segment (start 130.167 124.468) (end 130.167 130.063) (width 1.5) (layer B.Cu) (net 5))
 (segment (start 133.087 121.548) (end 130.167 124.468) (width 1.5) (layer B.Cu) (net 5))
 (segment (start 138.43 118.9105) (end 139.954 117.3865) (width 0.8) (layer B.Cu) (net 5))
 (segment (start 138.43 121.548) (end 138.43 118.9105) (width 0.8) (layer B.Cu) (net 5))
 (segment (start 134.468 115.824) (end 131.826 115.824) (width 0.8) (layer B.Cu) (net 4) (status 10))
 (segment (start 131.826 115.824) (end 128.168 115.824) (width 0.8) (layer B.Cu) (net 4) (status 20))
 (segment (start 132.015 108.545) (end 132.015 110.7905) (width 0.6) (layer B.Cu) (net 4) (status 30))
 (segment (start 130.48999 107.99499) (end 130.48999 102.38801) (width 0.6) (layer B.Cu) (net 4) (status 20))
 (segment (start 132.015 108.545) (end 131.04 108.545) (width 0.6) (layer B.Cu) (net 4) (status 30))
 (segment (start 131.04 108.545) (end 130.48999 107.99499) (width 0.6) (layer B.Cu) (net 4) (status 10))
 (segment (start 147.494 107.152) (end 144.816 107.152) (width 0.4) (layer B.Cu) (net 4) (status 30))
 (segment (start 147.494 106.502) (end 147.494 107.014) (width 0.4) (layer B.Cu) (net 4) (status 30))
 (segment (start 134.519 110.744) (end 135.1065 110.744) (width 0.8) (layer B.Cu) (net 4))
 (segment (start 132.817999 112.445001) (end 134.519 110.744) (width 0.8) (layer B.Cu) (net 4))
 (segment (start 132.817999 115.048001) (end 132.817999 112.445001) (width 0.8) (layer B.Cu) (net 4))
 (segment (start 133.847998 116.078) (end 132.817999 115.048001) (width 0.8) (layer B.Cu) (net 4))
 (segment (start 134.468 116.078) (end 133.847998 116.078) (width 0.8) (layer B.Cu) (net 4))
 (segment (start 132.0615 110.744) (end 131.5935 111.212) (width 0.6) (layer B.Cu) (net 4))
 (segment (start 135.1065 110.744) (end 132.0615 110.744) (width 0.6) (layer B.Cu) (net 4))
 (segment (start 143.9125 108.077) (end 144.78 107.2095) (width 0.6) (layer B.Cu) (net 4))
 (segment (start 135.1065 110.744) (end 137.7735 108.077) (width 0.6) (layer B.Cu) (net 4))
 (segment (start 137.7735 108.077) (end 143.9125 108.077) (width 0.6) (layer B.Cu) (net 4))
 (segment (start 124.1005 106.005) (end 123.444 106.6615) (width 0.4) (layer B.Cu) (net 7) (status 20))
 (segment (start 127.065 106.005) (end 124.1005 106.005) (width 0.4) (layer B.Cu) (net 7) (status 10))
 (segment (start 132.015 107.275) (end 139.765 107.275) (width 0.4) (layer B.Cu) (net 7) (status 10))
 (segment (start 139.765 107.275) (end 140.54 106.5) (width 0.4) (layer B.Cu) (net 7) (status 20))
 (segment (start 122.26899 100.459756) (end 122.26899 105.72899) (width 0.4) (layer B.Cu) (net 7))
 (segment (start 143.116 106.2736) (end 143.16601 106.22359) (width 0.4) (layer B.Cu) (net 7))
 (segment (start 140.716 106.2736) (end 143.116 106.2736) (width 0.4) (layer B.Cu) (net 7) (status 10))
 (segment (start 143.16601 100.592987) (end 140.071003 97.49798) (width 0.4) (layer B.Cu) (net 7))
 (segment (start 140.071003 97.49798) (end 125.230766 97.49798) (width 0.4) (layer B.Cu) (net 7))
 (segment (start 125.230766 97.49798) (end 122.26899 100.459756) (width 0.4) (layer B.Cu) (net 7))
 (segment (start 143.16601 106.22359) (end 143.16601 100.592987) (width 0.4) (layer B.Cu) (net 7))
 (segment (start 122.26899 105.72899) (end 123.04 106.5) (width 0.4) (layer B.Cu) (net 7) (status 20))
 (segment (start 123.04 106.5) (end 123.54 107) (width 0.4) (layer B.Cu) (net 7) (status 30))
 (segment (start 145.874966 105.842) (end 145.544966 106.172) (width 0.4) (layer B.Cu) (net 7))
 (segment (start 147.494 105.842) (end 145.874966 105.842) (width 0.4) (layer B.Cu) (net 7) (status 10))
 (segment (start 145.544966 106.172) (end 138.938 106.172) (width 0.4) (layer B.Cu) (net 7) (status 20))
 (segment (start 150.194 108.329) (end 147.652 110.871) (width 0.4) (layer B.Cu) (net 6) (status 20))
 (segment (start 150.194 107.152) (end 150.194 108.329) (width 0.4) (layer B.Cu) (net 6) (status 10))
 (segment (start 147.817998 119.38) (end 150.241 119.38) (width 0.6) (layer B.Cu) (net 6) (status 20))
 (segment (start 145.851999 117.414001) (end 147.817998 119.38) (width 0.6) (layer B.Cu) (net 6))
 (segment (start 145.851999 112.671001) (end 145.851999 117.414001) (width 0.6) (layer B.Cu) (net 6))
 (segment (start 147.652 110.871) (end 145.851999 112.671001) (width 0.6) (layer B.Cu) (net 6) (status 10))
 (segment (start 151.424001 106.552001) (end 151.424001 110.449999) (width 0.4) (layer B.Cu) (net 9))
 (segment (start 150.194 106.502) (end 151.374 106.502) (width 0.4) (layer B.Cu) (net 9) (status 10))
 (segment (start 151.374 106.502) (end 151.424001 106.552001) (width 0.4) (layer B.Cu) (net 9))
 (segment (start 147.652 114.222) (end 147.652 115.824) (width 0.4) (layer B.Cu) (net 9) (status 20))
 (segment (start 151.424001 110.449999) (end 147.652 114.222) (width 0.4) (layer B.Cu) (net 9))
 (segment (start 151.003 114.935) (end 151.003 115.824) (width 0.6) (layer B.Cu) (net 9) (status 10))
 (segment (start 151.003 115.824) (end 147.652 115.824) (width 0.6) (layer B.Cu) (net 9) (status 20))
 (segment (start 153.964 114.935) (end 156.464 112.435) (width 0.6) (layer B.Cu) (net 15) (status 20))
 (segment (start 152.828 114.935) (end 153.964 114.935) (width 0.6) (layer B.Cu) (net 15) (status 10))
 (segment (start 154.519 119.38) (end 156.464 117.435) (width 0.6) (layer B.Cu) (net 14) (status 20))
 (segment (start 152.066 119.38) (end 154.519 119.38) (width 0.6) (layer B.Cu) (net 14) (status 10))
 (segment (start 121.396 126.372) (end 125.087 130.063) (width 0.6) (layer B.Cu) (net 1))
 (segment (start 121.396 116.84) (end 121.396 126.372) (width 0.6) (layer B.Cu) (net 1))
 (segment (start 121.396 114.214) (end 121.396 116.84) (width 0.4) (layer B.Cu) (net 1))
 (segment (start 127.065 108.545) (end 121.396 114.214) (width 0.4) (layer B.Cu) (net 1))
 (segment (start 132.015 106.005) (end 135.001 106.005) (width 0.4) (layer B.Cu) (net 8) (status 30))
 (segment (start 135.001 106.005) (end 135.382 105.624) (width 0.4) (layer B.Cu) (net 8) (status 30))
 (segment (start 135.382 105.624) (end 135.89 106.132) (width 0.4) (layer B.Cu) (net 8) (status 30))
 (segment (start 140.716 103.7336) (end 137.8064 103.7336) (width 0.4) (layer B.Cu) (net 8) (status 10))
 (segment (start 137.8064 103.7336) (end 136.04 105.5) (width 0.4) (layer B.Cu) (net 8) (status 20))
 (segment (start 150.194 105.192) (end 150.194 104.194) (width 0.4) (layer B.Cu) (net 10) (status 10))
 (segment (start 119.618 105.934) (end 116.332 105.934) (width 0.4) (layer B.Cu) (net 10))
 (segment (start 150.194 103.966) (end 143.002 96.774) (width 0.4) (layer B.Cu) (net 10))
 (segment (start 150.194 104.194) (end 150.194 103.966) (width 0.4) (layer B.Cu) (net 10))
 (segment (start 143.002 96.774) (end 125.035494 96.774) (width 0.4) (layer B.Cu) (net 10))
 (segment (start 125.035494 96.774) (end 121.285 100.524494) (width 0.4) (layer B.Cu) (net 10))
 (segment (start 121.285 100.524494) (end 121.285 104.267) (width 0.4) (layer B.Cu) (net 10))
 (segment (start 121.285 104.267) (end 119.618 105.934) (width 0.4) (layer B.Cu) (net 10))
 (segment (start 116.332 107.934) (end 116.332 110.668) (width 0.6) (layer B.Cu) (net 13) (status 10))
 (segment (start 116.332 110.668) (end 115.5 111.5) (width 0.6) (layer B.Cu) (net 13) (status 20))
 (segment (start 115 116.8476) (end 118.8796 116.8476) (width 0.4) (layer B.Cu) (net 2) (status 30))
 (segment (start 118.8796 116.8476) (end 119.126 117.094) (width 0.4) (layer B.Cu) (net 2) (status 30))
 (segment (start 115.0076 116.84) (end 115 116.8476) (width 0.6) (layer B.Cu) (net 2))
 (segment (start 119.396 116.84) (end 115.0076 116.84) (width 0.6) (layer B.Cu) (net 2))
 (segment (start 119.0574 114.3076) (end 115 114.3076) (width 0.4) (layer B.Cu) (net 12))
 (segment (start 126.09 107.275) (end 119.0574 114.3076) (width 0.4) (layer B.Cu) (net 12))
 (segment (start 127.065 107.275) (end 126.09 107.275) (width 0.4) (layer B.Cu) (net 12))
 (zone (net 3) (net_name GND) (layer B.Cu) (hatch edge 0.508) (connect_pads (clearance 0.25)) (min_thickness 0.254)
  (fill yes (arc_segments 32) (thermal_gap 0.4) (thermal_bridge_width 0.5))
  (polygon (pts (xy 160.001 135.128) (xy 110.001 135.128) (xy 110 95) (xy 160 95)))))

